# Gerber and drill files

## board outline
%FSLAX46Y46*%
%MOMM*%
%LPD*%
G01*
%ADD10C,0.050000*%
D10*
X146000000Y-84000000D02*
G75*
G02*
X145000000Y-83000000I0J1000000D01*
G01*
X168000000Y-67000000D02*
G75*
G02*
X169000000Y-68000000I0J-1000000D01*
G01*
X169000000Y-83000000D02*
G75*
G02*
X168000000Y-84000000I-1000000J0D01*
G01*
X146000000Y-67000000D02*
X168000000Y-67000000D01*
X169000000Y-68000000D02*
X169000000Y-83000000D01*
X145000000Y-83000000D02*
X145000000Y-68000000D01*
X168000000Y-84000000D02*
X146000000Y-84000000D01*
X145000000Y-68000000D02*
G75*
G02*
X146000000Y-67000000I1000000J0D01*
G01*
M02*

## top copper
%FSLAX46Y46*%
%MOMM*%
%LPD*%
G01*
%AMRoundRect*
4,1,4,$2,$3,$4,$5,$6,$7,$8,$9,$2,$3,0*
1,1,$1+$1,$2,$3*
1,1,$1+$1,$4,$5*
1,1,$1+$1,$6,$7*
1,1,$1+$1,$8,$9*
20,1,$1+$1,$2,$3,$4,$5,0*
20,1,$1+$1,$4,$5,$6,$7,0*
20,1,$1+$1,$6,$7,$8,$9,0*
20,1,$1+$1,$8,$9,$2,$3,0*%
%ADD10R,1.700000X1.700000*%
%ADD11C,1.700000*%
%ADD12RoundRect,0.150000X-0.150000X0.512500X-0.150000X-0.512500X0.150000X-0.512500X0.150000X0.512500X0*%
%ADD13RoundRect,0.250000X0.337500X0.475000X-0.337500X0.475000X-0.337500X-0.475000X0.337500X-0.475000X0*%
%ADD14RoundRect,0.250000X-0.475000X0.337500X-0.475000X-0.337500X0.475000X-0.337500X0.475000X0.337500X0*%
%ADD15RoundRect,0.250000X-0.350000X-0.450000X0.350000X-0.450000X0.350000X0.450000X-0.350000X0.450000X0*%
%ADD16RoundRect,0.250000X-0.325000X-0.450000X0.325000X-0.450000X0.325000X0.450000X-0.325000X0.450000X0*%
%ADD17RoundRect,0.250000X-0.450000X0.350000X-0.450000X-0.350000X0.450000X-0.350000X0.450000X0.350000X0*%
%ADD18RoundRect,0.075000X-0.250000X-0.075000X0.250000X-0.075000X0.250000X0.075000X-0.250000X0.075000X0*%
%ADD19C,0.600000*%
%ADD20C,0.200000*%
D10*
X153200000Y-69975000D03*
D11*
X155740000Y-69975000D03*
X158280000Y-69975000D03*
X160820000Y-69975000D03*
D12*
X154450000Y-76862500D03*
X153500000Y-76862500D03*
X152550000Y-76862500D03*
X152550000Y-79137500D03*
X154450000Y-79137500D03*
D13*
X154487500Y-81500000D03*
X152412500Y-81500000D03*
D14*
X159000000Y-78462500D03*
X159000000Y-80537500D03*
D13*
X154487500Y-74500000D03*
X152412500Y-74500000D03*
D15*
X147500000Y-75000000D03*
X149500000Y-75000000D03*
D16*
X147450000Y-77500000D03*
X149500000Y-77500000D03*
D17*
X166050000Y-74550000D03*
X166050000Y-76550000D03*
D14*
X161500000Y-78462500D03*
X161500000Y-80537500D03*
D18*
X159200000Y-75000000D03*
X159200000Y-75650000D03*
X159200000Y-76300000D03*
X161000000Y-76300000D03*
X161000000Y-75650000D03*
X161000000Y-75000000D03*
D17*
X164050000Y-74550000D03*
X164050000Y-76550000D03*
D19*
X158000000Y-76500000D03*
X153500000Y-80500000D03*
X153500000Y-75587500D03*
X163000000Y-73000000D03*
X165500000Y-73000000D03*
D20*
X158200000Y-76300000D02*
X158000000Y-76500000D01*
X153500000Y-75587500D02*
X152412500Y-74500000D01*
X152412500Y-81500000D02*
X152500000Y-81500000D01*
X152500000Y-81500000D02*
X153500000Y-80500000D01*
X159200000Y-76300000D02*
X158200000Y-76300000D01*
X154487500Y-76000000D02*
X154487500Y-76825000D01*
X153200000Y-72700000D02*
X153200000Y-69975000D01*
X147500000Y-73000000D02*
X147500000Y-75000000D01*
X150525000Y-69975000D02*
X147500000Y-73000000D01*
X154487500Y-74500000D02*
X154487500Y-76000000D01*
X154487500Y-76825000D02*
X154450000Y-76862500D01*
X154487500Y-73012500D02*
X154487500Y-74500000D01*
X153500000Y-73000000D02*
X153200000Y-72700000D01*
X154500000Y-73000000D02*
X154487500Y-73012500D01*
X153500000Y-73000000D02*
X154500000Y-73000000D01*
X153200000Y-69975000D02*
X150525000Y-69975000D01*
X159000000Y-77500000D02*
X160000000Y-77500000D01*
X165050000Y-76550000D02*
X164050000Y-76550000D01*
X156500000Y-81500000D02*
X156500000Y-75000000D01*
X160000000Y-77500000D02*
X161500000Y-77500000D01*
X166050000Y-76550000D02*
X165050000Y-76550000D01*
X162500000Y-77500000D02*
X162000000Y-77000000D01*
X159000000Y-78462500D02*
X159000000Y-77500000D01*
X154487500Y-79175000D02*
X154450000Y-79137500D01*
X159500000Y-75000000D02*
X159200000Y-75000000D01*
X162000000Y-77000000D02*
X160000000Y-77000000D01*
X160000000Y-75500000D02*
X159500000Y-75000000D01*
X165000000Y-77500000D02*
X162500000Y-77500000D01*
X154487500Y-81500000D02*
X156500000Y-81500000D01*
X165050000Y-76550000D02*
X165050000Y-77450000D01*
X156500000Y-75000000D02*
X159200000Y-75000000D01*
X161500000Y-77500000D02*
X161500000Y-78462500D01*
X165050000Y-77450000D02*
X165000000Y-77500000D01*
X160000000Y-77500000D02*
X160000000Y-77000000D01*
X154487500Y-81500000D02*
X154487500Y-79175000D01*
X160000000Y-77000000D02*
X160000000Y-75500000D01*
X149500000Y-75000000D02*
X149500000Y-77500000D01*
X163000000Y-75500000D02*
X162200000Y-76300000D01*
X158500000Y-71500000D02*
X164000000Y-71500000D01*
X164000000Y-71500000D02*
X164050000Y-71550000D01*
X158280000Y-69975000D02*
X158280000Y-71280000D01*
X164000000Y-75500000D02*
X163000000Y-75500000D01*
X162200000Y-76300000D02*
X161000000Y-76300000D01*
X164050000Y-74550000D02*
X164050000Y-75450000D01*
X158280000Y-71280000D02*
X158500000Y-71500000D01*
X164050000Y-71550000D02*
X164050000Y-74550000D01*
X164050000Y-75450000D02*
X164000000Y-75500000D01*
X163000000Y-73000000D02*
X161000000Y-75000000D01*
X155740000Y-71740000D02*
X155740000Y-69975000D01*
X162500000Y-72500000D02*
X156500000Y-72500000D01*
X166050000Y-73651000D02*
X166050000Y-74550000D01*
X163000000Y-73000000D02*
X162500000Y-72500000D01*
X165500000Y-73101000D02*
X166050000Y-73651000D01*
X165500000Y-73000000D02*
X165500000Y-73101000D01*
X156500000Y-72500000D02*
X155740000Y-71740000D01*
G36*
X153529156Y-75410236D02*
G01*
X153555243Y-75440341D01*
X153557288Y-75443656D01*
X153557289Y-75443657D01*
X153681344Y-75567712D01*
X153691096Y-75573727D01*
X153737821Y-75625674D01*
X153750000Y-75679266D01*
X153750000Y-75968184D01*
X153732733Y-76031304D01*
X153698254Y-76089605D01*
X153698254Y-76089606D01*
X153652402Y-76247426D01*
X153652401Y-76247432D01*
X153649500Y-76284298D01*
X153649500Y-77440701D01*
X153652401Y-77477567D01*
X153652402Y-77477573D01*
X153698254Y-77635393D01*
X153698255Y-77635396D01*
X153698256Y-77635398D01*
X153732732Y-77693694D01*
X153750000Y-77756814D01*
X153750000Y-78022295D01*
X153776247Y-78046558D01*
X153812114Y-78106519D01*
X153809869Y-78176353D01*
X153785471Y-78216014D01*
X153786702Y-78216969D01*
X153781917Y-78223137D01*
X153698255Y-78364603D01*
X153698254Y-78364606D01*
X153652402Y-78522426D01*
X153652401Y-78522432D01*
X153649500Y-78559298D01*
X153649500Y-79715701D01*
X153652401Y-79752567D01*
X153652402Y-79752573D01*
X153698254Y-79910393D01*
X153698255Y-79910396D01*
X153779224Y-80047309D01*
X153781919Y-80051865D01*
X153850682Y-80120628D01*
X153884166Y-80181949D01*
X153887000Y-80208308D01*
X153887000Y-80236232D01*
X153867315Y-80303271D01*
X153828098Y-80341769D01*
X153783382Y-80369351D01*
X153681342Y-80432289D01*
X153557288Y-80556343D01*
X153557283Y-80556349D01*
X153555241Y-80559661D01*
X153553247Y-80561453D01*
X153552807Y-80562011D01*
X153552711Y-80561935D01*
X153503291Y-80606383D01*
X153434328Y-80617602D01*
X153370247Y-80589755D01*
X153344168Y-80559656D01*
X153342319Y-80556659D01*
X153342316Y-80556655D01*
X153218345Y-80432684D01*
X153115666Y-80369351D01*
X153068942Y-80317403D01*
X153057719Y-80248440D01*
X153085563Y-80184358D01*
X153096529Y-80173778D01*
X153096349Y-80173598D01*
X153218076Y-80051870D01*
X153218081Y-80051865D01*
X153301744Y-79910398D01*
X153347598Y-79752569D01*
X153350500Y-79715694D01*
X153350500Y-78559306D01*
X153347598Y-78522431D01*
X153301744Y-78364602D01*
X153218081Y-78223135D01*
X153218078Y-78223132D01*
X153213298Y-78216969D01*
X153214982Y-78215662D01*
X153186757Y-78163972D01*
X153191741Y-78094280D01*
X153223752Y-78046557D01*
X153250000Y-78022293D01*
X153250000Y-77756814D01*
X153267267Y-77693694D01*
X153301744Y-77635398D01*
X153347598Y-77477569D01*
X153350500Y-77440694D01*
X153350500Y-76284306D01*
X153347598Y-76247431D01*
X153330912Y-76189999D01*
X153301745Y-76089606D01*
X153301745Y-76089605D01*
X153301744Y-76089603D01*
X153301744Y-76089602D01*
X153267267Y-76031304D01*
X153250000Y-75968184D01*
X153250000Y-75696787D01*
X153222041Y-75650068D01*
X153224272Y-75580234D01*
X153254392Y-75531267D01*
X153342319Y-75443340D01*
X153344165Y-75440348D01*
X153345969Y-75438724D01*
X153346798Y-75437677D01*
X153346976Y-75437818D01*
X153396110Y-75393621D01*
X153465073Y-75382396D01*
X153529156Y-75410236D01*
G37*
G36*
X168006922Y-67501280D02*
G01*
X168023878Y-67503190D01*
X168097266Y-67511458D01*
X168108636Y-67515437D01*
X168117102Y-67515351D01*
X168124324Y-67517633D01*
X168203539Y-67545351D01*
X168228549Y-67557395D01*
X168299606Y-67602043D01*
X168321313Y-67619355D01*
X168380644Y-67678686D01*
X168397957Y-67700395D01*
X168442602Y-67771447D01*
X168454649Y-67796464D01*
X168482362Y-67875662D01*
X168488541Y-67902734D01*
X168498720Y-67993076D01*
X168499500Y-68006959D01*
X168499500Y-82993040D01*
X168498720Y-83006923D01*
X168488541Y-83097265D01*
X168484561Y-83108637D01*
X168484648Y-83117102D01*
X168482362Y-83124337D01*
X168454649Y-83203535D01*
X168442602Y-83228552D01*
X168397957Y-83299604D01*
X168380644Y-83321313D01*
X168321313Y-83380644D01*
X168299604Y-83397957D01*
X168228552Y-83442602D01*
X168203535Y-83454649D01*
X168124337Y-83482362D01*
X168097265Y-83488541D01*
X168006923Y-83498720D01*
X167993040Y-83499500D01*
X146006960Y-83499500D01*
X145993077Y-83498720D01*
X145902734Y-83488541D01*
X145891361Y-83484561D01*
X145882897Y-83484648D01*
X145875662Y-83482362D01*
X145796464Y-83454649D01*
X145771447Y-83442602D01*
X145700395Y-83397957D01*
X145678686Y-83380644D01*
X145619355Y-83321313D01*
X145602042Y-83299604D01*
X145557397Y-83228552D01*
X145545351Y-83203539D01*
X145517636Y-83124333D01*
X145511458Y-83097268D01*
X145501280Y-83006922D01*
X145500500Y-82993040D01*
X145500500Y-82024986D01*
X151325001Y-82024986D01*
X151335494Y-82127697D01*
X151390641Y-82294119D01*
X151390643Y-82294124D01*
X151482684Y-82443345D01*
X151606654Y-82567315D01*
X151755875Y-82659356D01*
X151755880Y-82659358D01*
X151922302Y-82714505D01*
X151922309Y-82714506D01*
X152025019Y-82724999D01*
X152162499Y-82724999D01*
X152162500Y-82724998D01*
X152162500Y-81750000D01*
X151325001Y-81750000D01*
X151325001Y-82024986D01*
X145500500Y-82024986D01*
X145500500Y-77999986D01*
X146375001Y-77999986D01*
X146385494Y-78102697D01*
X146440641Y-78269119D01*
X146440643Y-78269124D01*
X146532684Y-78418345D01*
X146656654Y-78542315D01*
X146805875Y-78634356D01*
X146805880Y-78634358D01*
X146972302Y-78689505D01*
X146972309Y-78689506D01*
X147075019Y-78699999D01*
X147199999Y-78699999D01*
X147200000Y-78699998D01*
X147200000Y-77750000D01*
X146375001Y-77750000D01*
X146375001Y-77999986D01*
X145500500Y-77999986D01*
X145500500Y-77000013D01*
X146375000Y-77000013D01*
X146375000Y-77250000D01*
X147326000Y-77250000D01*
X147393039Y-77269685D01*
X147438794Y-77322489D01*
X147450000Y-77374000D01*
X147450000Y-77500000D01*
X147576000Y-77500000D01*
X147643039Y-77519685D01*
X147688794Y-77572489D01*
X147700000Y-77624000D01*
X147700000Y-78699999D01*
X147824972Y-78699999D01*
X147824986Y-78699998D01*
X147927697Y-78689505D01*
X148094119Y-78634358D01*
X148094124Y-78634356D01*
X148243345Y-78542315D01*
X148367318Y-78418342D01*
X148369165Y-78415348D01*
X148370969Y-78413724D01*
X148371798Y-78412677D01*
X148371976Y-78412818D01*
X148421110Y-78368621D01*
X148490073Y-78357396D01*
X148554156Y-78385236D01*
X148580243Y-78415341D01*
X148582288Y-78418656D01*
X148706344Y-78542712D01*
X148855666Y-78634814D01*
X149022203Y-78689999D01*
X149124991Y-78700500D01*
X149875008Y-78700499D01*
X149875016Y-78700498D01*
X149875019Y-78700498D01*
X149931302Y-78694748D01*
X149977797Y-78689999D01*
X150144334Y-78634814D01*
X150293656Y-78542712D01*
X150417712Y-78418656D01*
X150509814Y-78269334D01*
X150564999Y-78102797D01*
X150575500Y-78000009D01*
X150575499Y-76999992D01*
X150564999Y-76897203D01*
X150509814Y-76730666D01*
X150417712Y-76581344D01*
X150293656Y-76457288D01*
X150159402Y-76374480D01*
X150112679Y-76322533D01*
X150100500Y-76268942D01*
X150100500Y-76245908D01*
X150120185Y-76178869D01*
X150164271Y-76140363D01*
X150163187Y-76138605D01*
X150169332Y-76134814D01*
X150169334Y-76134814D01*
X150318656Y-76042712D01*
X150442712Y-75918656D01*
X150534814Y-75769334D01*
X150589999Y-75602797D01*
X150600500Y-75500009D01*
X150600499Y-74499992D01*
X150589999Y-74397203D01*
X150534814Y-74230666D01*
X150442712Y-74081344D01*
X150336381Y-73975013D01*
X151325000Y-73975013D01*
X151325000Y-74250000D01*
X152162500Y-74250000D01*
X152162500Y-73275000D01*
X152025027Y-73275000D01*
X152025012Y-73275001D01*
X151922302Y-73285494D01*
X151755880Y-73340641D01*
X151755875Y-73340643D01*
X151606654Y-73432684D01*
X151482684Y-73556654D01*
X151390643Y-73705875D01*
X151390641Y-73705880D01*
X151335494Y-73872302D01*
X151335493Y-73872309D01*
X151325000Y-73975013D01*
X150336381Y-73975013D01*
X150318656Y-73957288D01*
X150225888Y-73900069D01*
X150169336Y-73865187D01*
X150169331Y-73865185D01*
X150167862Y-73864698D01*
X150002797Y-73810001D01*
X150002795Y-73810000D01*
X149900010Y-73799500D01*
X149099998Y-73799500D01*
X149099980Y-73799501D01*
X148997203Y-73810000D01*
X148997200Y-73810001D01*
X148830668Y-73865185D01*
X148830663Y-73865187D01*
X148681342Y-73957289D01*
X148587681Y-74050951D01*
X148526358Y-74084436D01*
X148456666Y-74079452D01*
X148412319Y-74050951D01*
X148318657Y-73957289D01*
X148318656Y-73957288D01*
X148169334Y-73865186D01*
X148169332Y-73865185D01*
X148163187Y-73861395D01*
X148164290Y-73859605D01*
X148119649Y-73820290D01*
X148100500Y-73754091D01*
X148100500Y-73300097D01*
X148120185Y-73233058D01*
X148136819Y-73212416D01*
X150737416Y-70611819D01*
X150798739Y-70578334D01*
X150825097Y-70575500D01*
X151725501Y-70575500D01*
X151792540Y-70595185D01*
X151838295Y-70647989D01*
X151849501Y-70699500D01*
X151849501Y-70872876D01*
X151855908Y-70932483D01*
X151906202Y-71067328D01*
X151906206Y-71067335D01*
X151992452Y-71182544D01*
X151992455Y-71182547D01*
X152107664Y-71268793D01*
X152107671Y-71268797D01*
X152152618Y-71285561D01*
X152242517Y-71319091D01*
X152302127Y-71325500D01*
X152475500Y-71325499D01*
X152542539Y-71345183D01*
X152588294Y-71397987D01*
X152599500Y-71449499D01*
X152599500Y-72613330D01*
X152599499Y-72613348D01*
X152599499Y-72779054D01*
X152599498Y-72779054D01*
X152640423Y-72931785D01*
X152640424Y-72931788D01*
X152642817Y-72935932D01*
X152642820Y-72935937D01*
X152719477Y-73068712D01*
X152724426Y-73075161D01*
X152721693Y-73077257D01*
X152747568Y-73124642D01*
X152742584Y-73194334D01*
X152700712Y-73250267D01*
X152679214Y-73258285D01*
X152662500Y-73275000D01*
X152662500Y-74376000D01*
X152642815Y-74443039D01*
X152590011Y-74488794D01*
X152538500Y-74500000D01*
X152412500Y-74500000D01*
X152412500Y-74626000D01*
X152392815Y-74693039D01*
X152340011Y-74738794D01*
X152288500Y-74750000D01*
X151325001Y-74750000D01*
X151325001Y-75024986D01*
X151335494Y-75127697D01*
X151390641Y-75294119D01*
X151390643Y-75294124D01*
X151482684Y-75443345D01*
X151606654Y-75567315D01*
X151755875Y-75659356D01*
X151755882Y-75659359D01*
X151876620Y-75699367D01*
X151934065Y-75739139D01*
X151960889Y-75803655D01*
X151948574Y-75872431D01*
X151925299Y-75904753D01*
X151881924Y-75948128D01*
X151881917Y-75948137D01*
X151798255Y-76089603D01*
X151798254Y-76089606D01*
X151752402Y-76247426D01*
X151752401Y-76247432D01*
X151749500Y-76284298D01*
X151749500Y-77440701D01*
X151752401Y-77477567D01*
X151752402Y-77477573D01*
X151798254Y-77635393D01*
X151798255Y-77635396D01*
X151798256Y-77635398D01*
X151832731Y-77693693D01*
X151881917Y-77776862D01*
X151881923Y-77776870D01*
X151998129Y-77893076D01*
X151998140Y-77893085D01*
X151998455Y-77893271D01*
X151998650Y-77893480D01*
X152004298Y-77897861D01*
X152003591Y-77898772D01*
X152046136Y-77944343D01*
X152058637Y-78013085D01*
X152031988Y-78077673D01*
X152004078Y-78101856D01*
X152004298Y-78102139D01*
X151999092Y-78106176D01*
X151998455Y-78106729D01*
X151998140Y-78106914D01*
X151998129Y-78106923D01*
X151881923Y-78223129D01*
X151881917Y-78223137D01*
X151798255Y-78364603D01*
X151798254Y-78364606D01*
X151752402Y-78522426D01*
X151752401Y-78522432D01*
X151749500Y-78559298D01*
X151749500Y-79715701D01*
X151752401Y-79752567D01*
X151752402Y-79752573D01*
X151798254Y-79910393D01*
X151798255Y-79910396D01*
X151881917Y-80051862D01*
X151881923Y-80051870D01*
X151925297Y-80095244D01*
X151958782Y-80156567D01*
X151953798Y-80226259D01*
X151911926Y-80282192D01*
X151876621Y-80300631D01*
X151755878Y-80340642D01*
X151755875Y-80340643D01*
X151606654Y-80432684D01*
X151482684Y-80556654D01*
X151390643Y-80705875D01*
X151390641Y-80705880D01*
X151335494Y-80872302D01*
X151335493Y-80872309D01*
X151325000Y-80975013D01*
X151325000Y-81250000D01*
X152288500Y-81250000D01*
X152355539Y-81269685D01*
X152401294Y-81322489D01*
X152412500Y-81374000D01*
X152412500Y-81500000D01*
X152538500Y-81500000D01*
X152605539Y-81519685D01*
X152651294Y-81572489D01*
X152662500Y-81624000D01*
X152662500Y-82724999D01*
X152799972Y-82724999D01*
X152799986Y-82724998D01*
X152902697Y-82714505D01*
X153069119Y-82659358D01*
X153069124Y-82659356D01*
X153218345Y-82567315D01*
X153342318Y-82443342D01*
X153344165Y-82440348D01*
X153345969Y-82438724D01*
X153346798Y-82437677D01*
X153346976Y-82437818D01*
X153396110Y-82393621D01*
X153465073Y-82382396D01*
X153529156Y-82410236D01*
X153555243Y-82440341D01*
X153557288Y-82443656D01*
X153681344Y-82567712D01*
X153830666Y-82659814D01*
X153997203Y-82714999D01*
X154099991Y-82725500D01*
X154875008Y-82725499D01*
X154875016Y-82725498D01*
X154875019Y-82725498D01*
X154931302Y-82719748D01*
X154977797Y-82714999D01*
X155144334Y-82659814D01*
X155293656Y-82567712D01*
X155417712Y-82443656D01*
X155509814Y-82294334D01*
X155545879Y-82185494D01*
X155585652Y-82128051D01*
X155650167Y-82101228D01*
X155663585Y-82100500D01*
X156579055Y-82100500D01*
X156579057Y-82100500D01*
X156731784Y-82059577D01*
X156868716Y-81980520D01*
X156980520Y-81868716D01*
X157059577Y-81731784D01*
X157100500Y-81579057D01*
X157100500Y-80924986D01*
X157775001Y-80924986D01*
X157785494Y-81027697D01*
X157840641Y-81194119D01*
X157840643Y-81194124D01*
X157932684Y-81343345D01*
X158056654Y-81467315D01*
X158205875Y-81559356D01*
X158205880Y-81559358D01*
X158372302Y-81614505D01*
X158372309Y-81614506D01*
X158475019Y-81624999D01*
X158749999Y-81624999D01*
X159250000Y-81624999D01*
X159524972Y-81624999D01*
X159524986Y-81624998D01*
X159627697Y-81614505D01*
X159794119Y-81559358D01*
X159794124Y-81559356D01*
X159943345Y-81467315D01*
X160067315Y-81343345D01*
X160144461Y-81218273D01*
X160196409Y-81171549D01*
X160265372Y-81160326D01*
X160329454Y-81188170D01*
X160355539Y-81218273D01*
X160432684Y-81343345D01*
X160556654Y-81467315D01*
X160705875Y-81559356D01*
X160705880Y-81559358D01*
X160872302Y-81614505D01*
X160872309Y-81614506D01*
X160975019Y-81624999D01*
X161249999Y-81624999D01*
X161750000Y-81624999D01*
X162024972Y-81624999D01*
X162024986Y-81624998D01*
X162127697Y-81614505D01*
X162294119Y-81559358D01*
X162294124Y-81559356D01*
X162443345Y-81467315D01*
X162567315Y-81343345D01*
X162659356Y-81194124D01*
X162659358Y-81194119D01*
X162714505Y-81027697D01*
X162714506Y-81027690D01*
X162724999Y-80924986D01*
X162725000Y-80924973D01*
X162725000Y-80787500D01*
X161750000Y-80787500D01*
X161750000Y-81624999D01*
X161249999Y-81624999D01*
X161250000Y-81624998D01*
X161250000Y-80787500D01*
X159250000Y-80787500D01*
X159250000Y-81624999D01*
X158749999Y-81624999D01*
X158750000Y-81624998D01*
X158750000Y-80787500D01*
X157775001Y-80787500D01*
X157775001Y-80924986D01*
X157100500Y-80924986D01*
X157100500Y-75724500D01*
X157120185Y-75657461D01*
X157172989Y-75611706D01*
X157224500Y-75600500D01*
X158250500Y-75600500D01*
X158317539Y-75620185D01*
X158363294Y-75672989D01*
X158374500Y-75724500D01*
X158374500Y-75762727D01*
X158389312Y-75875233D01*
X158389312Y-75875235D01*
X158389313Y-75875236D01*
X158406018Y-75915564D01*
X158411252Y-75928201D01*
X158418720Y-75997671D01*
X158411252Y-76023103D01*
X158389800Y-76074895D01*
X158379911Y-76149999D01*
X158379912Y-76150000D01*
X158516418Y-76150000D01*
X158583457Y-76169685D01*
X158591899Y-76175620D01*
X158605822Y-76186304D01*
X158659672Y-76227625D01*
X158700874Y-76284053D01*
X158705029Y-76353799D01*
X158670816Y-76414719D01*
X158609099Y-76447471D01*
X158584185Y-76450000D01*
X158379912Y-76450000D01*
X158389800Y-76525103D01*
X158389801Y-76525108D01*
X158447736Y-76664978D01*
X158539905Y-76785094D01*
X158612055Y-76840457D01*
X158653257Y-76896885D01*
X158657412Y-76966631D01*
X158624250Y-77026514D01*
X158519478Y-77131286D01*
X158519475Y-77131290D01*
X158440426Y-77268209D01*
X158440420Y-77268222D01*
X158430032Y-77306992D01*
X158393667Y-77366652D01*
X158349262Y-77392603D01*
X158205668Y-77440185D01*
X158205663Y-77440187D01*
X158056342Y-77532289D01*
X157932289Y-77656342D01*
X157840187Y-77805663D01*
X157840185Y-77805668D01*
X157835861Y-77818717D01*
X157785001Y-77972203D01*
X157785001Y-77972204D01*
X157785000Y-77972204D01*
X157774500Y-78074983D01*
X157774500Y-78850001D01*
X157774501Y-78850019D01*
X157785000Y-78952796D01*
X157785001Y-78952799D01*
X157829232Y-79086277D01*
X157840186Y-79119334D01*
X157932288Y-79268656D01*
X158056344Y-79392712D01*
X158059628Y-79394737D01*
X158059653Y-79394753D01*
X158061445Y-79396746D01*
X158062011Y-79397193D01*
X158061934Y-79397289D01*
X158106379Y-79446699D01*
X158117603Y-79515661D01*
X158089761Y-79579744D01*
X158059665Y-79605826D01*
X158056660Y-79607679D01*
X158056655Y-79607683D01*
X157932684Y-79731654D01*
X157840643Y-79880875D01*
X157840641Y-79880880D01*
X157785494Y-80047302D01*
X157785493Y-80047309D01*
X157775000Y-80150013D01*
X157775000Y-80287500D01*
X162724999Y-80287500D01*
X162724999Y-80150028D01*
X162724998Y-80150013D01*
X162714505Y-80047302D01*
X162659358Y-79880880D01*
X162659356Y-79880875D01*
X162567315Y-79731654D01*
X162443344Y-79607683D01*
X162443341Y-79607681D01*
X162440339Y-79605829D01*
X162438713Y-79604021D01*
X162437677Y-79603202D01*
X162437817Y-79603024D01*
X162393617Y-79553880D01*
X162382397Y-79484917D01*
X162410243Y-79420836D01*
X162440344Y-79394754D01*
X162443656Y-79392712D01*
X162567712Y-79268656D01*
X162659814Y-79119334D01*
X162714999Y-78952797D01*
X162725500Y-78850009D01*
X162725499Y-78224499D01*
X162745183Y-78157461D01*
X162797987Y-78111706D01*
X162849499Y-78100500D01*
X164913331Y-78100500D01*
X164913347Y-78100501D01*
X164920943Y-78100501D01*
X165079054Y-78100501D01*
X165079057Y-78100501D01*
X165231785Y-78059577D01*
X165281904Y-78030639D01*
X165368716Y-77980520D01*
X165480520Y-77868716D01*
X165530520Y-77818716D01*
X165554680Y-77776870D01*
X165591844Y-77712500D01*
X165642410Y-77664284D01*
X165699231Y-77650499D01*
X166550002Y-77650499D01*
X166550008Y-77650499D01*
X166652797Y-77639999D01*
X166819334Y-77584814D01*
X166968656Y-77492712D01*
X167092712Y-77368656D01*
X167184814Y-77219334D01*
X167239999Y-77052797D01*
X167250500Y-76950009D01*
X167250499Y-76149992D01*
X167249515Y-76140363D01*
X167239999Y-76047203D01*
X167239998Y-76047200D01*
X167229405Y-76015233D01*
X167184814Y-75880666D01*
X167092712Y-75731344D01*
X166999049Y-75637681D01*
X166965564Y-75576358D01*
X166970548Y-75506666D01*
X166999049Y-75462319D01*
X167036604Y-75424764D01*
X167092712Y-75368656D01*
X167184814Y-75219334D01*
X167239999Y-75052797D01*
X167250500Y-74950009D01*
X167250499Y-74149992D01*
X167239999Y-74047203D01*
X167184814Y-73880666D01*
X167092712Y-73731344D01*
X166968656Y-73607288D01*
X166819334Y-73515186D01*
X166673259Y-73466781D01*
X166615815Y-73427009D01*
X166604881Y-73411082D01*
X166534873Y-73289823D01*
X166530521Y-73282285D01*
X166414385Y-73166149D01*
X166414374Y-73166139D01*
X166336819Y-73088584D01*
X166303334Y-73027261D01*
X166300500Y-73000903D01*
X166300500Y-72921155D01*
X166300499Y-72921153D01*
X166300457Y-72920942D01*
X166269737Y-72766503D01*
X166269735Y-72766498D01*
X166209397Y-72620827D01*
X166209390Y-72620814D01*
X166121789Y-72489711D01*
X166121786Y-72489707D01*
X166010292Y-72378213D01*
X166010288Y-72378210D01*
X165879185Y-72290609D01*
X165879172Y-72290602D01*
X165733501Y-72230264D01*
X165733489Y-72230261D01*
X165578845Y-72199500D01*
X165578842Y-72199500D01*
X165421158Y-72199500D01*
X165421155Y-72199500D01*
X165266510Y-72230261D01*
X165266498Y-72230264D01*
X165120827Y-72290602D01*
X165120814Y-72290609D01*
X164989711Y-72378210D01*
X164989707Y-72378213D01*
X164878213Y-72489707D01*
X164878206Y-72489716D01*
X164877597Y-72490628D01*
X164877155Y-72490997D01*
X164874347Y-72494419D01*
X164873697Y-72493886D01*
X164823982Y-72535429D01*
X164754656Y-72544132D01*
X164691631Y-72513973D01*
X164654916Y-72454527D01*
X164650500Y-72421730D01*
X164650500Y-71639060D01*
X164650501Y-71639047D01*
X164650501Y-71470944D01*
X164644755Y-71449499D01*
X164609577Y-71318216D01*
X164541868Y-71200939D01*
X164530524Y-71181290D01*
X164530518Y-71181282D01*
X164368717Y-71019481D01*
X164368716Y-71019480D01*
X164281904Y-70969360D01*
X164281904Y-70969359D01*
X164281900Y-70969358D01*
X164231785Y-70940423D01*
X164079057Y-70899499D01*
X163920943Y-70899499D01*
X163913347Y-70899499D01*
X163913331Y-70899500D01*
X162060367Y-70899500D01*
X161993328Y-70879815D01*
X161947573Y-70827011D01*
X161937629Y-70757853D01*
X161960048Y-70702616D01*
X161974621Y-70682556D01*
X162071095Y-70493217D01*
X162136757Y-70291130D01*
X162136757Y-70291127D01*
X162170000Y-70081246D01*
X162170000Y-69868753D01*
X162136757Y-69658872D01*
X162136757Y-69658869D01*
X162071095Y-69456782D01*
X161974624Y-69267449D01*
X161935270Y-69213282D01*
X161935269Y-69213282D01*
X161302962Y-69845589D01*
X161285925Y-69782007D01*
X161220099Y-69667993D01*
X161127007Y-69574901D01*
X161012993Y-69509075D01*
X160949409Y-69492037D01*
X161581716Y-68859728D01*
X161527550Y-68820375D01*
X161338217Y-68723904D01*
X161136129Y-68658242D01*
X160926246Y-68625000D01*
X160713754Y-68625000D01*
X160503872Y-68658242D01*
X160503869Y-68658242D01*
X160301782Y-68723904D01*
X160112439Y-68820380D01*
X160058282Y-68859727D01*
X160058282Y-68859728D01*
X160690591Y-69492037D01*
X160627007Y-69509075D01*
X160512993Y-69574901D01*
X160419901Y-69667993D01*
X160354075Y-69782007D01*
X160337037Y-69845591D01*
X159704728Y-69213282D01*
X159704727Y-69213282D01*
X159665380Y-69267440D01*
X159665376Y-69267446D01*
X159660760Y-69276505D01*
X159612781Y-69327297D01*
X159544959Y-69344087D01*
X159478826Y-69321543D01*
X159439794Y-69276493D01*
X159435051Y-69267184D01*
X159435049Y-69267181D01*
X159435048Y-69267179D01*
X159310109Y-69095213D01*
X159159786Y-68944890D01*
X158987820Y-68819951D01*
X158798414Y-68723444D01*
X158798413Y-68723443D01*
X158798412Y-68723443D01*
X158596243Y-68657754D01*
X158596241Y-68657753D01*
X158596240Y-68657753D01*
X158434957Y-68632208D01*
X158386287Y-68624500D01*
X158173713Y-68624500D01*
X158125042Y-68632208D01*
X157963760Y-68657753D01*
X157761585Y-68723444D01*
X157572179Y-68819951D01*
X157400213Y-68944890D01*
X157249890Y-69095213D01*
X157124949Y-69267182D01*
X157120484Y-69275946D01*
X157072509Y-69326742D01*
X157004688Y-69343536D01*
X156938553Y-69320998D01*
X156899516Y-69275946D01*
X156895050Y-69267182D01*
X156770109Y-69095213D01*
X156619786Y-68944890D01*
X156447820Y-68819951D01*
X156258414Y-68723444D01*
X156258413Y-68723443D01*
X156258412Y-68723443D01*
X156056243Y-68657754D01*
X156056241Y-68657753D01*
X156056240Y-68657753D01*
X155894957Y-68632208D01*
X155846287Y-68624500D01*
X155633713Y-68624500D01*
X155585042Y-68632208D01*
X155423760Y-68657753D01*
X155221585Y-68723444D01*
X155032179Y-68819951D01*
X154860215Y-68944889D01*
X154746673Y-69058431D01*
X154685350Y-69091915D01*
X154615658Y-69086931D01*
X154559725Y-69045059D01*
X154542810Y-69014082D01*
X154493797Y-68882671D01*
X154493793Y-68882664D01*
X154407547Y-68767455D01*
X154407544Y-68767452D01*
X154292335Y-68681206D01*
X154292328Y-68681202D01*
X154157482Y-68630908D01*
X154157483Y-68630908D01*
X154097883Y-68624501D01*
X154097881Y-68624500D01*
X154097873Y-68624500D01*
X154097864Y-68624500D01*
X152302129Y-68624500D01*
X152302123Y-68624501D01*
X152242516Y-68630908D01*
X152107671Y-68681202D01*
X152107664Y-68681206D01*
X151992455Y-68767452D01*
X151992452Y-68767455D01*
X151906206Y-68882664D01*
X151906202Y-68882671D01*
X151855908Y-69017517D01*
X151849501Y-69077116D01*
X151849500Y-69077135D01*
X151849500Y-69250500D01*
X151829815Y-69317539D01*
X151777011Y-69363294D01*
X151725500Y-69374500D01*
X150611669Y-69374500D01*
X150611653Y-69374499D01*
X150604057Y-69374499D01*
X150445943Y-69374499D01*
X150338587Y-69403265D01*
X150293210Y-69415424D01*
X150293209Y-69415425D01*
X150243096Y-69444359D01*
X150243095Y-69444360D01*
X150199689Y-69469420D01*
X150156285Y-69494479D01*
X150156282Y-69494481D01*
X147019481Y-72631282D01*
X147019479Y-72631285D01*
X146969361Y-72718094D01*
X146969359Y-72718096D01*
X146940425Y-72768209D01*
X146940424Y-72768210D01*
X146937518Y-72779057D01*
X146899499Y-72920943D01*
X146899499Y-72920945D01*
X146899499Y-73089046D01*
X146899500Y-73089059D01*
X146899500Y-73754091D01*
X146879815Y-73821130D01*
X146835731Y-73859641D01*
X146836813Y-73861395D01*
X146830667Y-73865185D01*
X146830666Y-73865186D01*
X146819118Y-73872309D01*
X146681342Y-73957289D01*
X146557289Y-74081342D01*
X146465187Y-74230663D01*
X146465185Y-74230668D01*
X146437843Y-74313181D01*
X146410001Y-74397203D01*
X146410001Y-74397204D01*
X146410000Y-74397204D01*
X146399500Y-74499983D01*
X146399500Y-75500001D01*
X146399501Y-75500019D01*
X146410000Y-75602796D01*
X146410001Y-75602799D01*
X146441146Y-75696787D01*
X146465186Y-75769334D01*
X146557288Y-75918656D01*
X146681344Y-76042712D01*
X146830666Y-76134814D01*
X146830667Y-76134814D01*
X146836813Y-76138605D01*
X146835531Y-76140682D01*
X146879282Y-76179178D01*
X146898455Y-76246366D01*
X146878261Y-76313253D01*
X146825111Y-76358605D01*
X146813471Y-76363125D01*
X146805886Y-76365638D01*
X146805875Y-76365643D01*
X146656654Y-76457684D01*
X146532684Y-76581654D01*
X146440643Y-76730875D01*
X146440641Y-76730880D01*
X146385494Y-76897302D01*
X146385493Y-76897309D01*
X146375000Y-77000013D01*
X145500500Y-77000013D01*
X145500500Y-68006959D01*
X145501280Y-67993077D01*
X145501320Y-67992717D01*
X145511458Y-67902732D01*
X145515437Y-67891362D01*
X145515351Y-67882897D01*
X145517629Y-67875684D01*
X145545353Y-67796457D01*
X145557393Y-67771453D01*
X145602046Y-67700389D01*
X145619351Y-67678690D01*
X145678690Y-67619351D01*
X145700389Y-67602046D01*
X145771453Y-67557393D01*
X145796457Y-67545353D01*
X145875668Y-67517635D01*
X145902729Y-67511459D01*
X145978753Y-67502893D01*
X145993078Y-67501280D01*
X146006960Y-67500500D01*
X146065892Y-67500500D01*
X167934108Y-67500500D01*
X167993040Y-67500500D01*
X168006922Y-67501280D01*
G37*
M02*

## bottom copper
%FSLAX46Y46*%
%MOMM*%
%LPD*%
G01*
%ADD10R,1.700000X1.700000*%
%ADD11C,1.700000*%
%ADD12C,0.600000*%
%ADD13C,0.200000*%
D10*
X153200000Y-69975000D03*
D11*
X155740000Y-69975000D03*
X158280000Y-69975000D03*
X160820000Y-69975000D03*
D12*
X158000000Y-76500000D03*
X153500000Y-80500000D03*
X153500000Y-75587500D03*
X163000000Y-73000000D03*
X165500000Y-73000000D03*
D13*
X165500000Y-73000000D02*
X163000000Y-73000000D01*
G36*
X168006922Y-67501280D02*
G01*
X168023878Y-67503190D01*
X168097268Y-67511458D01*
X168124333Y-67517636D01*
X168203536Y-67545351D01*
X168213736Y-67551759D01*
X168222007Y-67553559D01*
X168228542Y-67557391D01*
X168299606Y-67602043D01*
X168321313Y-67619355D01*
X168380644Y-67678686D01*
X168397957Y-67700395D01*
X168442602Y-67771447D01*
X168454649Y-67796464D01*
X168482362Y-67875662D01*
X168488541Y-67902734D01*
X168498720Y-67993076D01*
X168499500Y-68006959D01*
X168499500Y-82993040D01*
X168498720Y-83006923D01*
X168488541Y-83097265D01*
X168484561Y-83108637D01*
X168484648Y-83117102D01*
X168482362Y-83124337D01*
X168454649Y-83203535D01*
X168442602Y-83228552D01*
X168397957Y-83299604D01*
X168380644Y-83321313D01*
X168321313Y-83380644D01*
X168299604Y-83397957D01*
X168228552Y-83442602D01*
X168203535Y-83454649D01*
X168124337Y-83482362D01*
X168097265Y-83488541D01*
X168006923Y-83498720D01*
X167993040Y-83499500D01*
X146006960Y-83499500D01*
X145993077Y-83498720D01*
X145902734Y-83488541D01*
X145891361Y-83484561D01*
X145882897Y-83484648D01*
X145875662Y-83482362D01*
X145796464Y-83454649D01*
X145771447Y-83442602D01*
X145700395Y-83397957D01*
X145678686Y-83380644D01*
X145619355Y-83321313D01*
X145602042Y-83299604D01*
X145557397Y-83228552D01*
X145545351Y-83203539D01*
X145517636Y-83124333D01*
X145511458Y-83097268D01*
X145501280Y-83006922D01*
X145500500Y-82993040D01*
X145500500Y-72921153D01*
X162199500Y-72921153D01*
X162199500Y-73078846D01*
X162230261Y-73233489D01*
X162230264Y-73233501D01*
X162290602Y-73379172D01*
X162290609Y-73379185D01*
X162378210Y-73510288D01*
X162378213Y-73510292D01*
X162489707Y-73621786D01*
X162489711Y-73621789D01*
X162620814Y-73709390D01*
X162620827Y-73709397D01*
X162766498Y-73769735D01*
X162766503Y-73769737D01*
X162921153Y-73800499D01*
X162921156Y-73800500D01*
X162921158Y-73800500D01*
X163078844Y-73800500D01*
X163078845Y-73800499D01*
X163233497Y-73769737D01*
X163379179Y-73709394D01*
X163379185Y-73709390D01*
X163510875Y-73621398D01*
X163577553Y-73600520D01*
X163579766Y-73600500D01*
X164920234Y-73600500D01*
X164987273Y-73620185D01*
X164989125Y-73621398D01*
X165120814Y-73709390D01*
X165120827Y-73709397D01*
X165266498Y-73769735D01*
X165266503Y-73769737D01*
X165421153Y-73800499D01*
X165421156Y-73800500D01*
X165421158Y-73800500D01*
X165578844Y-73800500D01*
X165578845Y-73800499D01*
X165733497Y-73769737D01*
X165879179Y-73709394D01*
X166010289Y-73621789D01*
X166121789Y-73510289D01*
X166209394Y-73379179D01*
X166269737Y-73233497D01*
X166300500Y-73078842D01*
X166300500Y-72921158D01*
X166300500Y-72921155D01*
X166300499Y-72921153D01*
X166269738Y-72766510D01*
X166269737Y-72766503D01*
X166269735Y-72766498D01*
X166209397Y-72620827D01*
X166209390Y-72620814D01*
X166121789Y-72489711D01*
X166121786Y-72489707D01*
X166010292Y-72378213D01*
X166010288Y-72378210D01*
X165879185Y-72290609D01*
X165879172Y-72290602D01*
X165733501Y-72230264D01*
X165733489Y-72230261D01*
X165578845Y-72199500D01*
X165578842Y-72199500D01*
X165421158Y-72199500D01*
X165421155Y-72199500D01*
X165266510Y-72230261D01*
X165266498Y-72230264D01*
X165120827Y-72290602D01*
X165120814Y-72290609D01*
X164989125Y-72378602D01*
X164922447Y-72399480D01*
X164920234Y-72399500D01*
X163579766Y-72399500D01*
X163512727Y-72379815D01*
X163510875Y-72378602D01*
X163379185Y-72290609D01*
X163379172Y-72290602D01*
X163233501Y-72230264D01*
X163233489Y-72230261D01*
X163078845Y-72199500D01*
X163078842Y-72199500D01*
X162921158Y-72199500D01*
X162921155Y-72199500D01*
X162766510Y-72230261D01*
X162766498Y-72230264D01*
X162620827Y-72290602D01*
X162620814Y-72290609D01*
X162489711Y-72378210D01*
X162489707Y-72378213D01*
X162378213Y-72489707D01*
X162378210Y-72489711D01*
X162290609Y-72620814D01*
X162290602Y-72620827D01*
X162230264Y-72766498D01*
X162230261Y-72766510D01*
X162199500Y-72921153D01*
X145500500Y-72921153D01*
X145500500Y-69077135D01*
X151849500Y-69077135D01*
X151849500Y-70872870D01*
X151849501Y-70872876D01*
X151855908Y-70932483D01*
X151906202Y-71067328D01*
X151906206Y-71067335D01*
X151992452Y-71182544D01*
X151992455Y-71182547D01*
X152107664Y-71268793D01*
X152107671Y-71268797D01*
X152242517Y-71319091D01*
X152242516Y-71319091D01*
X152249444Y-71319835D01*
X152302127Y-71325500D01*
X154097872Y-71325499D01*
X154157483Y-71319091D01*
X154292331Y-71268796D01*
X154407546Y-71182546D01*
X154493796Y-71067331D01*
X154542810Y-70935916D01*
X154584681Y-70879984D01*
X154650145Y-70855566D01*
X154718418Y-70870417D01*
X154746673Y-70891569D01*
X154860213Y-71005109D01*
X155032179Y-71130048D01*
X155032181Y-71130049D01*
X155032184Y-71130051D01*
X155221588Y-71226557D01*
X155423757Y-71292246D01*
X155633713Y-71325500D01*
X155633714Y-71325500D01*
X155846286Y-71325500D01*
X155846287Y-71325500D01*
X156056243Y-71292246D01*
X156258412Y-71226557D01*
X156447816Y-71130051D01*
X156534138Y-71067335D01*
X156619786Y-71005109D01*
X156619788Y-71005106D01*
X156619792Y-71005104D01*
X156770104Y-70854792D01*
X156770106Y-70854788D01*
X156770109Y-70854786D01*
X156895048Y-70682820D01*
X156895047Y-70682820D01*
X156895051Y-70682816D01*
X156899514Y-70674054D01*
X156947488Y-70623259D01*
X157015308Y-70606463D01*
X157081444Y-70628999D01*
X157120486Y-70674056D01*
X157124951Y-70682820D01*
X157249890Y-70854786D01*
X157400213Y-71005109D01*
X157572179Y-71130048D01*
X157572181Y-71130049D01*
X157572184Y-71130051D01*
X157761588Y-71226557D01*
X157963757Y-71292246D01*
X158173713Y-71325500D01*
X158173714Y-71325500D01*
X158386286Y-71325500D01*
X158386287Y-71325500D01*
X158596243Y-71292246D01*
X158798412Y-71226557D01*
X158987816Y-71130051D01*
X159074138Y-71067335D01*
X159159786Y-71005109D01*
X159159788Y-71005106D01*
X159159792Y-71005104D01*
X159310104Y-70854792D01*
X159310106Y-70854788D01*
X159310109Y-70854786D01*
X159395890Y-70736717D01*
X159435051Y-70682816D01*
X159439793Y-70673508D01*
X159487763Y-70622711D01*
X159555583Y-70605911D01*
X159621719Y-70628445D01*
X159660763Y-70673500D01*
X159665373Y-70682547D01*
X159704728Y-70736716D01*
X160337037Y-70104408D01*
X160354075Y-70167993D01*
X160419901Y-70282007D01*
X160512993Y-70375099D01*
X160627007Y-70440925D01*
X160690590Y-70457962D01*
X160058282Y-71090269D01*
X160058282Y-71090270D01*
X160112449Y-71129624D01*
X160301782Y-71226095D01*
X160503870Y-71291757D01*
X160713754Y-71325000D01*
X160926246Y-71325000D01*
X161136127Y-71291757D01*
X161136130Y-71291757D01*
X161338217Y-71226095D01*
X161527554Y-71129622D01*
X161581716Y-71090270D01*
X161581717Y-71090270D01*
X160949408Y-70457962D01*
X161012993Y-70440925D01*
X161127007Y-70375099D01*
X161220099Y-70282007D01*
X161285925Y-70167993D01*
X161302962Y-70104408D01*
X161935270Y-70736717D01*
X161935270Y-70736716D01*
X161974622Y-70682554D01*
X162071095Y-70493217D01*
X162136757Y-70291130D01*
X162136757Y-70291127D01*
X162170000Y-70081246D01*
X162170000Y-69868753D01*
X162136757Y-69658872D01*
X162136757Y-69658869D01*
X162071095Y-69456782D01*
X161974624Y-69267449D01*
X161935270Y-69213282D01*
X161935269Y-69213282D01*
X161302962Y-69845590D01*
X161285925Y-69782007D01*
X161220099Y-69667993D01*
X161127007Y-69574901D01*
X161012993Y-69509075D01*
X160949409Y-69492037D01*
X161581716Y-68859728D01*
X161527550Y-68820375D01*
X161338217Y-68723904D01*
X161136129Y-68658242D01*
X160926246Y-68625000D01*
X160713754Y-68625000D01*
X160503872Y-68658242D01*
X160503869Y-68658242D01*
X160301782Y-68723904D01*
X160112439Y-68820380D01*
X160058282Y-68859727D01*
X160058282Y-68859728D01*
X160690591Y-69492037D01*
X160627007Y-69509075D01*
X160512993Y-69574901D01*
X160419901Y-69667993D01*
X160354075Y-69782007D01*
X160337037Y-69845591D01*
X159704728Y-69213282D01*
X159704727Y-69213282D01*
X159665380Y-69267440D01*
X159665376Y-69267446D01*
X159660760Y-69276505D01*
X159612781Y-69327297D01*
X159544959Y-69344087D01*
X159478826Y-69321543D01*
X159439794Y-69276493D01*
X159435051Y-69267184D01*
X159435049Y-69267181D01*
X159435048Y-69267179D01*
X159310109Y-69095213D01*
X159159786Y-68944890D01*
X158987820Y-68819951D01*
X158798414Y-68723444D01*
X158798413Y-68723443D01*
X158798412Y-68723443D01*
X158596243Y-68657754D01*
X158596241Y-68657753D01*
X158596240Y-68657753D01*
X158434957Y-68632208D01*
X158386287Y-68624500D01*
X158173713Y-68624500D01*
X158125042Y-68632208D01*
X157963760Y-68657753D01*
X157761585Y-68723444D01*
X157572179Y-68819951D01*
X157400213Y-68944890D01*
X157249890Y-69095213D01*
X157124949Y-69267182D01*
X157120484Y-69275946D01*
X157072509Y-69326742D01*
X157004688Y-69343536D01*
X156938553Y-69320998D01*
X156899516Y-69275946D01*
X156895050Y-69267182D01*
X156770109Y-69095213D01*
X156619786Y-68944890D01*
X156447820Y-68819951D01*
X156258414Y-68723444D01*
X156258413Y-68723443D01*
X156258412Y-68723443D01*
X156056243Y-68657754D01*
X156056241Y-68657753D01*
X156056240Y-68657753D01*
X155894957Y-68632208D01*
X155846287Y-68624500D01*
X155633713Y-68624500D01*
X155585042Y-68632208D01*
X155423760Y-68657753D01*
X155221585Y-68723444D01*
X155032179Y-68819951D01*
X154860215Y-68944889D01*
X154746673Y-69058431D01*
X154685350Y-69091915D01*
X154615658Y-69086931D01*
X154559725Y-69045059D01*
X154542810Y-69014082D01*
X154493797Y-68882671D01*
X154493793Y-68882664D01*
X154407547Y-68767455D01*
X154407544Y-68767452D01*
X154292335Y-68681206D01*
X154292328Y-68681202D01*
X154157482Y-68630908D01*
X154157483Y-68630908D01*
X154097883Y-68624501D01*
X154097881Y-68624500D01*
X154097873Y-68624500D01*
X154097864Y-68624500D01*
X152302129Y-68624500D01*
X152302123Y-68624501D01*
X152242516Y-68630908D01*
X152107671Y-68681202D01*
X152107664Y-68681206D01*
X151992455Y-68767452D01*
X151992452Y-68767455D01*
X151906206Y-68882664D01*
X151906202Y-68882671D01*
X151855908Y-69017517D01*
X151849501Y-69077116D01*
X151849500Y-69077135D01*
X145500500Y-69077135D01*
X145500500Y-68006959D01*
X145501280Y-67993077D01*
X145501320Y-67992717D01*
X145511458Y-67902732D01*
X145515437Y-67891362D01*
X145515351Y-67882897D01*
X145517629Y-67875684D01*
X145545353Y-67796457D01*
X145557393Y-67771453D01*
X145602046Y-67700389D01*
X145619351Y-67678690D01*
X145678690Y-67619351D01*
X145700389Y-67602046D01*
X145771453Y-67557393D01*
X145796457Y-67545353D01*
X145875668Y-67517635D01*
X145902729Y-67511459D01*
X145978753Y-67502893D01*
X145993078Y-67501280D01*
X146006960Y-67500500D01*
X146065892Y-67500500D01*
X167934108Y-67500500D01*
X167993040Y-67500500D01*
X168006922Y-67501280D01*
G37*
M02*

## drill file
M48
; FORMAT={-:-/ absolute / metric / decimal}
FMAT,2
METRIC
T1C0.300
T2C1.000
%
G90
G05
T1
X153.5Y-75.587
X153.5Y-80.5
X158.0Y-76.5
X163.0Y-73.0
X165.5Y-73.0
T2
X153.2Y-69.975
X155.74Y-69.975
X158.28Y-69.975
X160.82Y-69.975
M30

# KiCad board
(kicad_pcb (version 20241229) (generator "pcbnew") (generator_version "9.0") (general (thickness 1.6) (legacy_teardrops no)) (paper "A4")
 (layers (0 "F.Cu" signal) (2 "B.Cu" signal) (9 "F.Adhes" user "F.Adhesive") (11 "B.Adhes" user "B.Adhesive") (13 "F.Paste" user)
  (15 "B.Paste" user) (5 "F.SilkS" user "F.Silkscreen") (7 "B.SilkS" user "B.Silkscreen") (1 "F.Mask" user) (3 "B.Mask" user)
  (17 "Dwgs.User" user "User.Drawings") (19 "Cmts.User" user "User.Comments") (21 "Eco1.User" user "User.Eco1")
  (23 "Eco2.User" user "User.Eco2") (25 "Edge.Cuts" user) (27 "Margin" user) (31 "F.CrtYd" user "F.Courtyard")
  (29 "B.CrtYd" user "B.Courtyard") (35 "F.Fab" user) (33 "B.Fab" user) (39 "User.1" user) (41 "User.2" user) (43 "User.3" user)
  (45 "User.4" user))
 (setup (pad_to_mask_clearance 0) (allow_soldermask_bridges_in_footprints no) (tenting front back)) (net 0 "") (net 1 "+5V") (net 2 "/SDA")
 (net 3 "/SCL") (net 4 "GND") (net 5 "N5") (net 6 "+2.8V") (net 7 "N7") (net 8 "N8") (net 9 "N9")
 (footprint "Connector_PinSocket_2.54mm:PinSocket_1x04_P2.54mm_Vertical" (layer "F.Cu") (at 153.2 69.975 90)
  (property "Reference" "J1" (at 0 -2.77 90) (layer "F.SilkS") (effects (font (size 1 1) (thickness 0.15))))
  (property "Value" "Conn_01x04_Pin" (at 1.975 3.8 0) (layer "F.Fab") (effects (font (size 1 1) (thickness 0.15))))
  (pad "1" thru_hole rect (at 0 0 90) (size 1.7 1.7) (drill 1) (layers "*.Cu" "*.Mask") (remove_unused_layers no) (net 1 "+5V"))
  (pad "2" thru_hole circle (at 0 2.54 90) (size 1.7 1.7) (drill 1) (layers "*.Cu" "*.Mask") (remove_unused_layers no) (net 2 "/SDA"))
  (pad "3" thru_hole circle (at 0 5.08 90) (size 1.7 1.7) (drill 1) (layers "*.Cu" "*.Mask") (remove_unused_layers no) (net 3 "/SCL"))
  (pad "4" thru_hole circle (at 0 7.62 90) (size 1.7 1.7) (drill 1) (layers "*.Cu" "*.Mask") (remove_unused_layers no) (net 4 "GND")))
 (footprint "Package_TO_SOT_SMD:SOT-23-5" (layer "F.Cu") (at 153.5 78 -90)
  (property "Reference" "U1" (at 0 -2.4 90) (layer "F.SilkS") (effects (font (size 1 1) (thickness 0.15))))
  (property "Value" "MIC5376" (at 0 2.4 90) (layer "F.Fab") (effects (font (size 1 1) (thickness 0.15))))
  (pad "1" smd roundrect (at -1.1375 -0.95 270) (size 1.325 0.6) (layers "F.Cu" "F.Mask" "F.Paste") (roundrect_rratio 0.25) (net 1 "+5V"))
  (pad "2" smd roundrect (at -1.1375 0 270) (size 1.325 0.6) (layers "F.Cu" "F.Mask" "F.Paste") (roundrect_rratio 0.25) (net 4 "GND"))
  (pad "3" smd roundrect (at -1.1375 0.95 270) (size 1.325 0.6) (layers "F.Cu" "F.Mask" "F.Paste") (roundrect_rratio 0.25) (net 1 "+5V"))
  (pad "4" smd roundrect (at 1.1375 0.95 270) (size 1.325 0.6) (layers "F.Cu" "F.Mask" "F.Paste") (roundrect_rratio 0.25) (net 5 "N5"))
  (pad "5" smd roundrect (at 1.1375 -0.95 270) (size 1.325 0.6) (layers "F.Cu" "F.Mask" "F.Paste") (roundrect_rratio 0.25) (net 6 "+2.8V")))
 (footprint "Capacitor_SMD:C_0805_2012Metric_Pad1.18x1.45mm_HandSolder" (layer "F.Cu") (at 153.45 81.5 180)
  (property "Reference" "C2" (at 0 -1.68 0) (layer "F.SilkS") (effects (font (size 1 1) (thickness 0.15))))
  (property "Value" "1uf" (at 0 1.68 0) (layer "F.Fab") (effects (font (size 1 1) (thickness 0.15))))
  (pad "1" smd roundrect (at -1.0375 0 180) (size 1.175 1.45) (layers "F.Cu" "F.Mask" "F.Paste") (roundrect_rratio 0.212766) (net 6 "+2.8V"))
  (pad "2" smd roundrect (at 1.0375 0 180) (size 1.175 1.45) (layers "F.Cu" "F.Mask" "F.Paste") (roundrect_rratio 0.212766) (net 4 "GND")))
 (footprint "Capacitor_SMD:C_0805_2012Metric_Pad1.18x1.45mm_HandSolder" (layer "F.Cu") (at 159 79.5 -90)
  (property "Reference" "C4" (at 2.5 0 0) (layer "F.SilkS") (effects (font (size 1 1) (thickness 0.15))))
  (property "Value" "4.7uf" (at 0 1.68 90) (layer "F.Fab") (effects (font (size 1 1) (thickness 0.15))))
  (pad "1" smd roundrect (at -1.0375 0 270) (size 1.175 1.45) (layers "F.Cu" "F.Mask" "F.Paste") (roundrect_rratio 0.212766) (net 6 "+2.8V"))
  (pad "2" smd roundrect (at 1.0375 0 270) (size 1.175 1.45) (layers "F.Cu" "F.Mask" "F.Paste") (roundrect_rratio 0.212766) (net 4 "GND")))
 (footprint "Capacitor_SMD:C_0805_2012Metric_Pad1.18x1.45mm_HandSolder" (layer "F.Cu") (at 153.45 74.5 180)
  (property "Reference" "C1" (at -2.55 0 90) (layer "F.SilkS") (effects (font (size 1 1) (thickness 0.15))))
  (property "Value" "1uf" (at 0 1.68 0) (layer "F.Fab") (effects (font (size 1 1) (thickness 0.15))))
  (pad "1" smd roundrect (at -1.0375 0 180) (size 1.175 1.45) (layers "F.Cu" "F.Mask" "F.Paste") (roundrect_rratio 0.212766) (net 1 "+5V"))
  (pad "2" smd roundrect (at 1.0375 0 180) (size 1.175 1.45) (layers "F.Cu" "F.Mask" "F.Paste") (roundrect_rratio 0.212766) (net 4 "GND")))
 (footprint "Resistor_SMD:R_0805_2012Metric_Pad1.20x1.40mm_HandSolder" (layer "F.Cu") (at 148.5 75)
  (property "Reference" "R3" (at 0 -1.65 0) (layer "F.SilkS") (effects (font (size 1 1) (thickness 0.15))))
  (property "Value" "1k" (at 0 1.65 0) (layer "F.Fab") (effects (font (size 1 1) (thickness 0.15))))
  (pad "1" smd roundrect (at -1 0) (size 1.2 1.4) (layers "F.Cu" "F.Mask" "F.Paste") (roundrect_rratio 0.208333) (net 1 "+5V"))
  (pad "2" smd roundrect (at 1 0) (size 1.2 1.4) (layers "F.Cu" "F.Mask" "F.Paste") (roundrect_rratio 0.208333) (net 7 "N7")))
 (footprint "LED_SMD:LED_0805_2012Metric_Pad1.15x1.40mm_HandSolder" (layer "F.Cu") (at 148.475 77.5)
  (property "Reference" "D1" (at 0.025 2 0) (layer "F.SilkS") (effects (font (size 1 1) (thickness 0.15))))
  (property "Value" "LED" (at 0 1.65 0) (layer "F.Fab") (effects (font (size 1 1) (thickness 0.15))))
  (pad "1" smd roundrect (at -1.025 0) (size 1.15 1.4) (layers "F.Cu" "F.Mask" "F.Paste") (roundrect_rratio 0.217391) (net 4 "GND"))
  (pad "2" smd roundrect (at 1.025 0) (size 1.15 1.4) (layers "F.Cu" "F.Mask" "F.Paste") (roundrect_rratio 0.217391) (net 7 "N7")))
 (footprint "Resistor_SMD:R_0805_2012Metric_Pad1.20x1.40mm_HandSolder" (layer "F.Cu") (at 166.05 75.55 -90)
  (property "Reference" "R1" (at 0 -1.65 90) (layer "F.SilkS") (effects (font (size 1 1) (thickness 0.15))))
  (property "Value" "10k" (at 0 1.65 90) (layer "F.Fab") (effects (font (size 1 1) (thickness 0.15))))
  (pad "1" smd roundrect (at -1 0 270) (size 1.2 1.4) (layers "F.Cu" "F.Mask" "F.Paste") (roundrect_rratio 0.208333) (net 2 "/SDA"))
  (pad "2" smd roundrect (at 1 0 270) (size 1.2 1.4) (layers "F.Cu" "F.Mask" "F.Paste") (roundrect_rratio 0.208333) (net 6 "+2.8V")))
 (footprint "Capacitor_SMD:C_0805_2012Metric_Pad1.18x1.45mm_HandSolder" (layer "F.Cu") (at 161.5 79.5 -90)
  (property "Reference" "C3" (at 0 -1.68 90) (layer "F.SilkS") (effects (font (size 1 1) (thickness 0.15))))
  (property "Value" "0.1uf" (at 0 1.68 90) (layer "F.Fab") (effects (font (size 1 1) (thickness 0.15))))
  (pad "1" smd roundrect (at -1.0375 0 270) (size 1.175 1.45) (layers "F.Cu" "F.Mask" "F.Paste") (roundrect_rratio 0.212766) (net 6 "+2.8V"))
  (pad "2" smd roundrect (at 1.0375 0 270) (size 1.175 1.45) (layers "F.Cu" "F.Mask" "F.Paste") (roundrect_rratio 0.212766) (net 4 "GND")))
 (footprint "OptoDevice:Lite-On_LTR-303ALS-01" (layer "F.Cu") (at 160.1 75.65)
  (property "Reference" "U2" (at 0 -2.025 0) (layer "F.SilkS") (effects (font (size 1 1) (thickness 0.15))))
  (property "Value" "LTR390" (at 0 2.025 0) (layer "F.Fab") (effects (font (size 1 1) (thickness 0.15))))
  (pad "1" smd roundrect (at -0.9 -0.65) (size 0.65 0.3) (layers "F.Cu" "F.Mask" "F.Paste") (roundrect_rratio 0.25) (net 6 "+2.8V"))
  (pad "2" smd roundrect (at -0.9 0) (size 0.65 0.3) (layers "F.Cu" "F.Mask" "F.Paste") (roundrect_rratio 0.25) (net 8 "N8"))
  (pad "3" smd roundrect (at -0.9 0.65) (size 0.65 0.3) (layers "F.Cu" "F.Mask" "F.Paste") (roundrect_rratio 0.25) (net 4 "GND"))
  (pad "4" smd roundrect (at 0.9 0.65) (size 0.65 0.3) (layers "F.Cu" "F.Mask" "F.Paste") (roundrect_rratio 0.25) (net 3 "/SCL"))
  (pad "5" smd roundrect (at 0.9 0) (size 0.65 0.3) (layers "F.Cu" "F.Mask" "F.Paste") (roundrect_rratio 0.25) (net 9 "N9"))
  (pad "6" smd roundrect (at 0.9 -0.65) (size 0.65 0.3) (layers "F.Cu" "F.Mask" "F.Paste") (roundrect_rratio 0.25) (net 2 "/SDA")))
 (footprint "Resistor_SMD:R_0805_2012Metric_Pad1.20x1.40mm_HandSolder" (layer "F.Cu") (at 164.05 75.55 -90)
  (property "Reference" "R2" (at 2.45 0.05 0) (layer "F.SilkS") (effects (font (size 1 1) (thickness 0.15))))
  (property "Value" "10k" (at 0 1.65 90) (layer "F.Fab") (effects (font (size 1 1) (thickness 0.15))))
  (pad "1" smd roundrect (at -1 0 270) (size 1.2 1.4) (layers "F.Cu" "F.Mask" "F.Paste") (roundrect_rratio 0.208333) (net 3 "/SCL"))
  (pad "2" smd roundrect (at 1 0 270) (size 1.2 1.4) (layers "F.Cu" "F.Mask" "F.Paste") (roundrect_rratio 0.208333) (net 6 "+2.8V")))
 (gr_arc (start 146 84) (mid 145.292893 83.707107) (end 145 83) (stroke (width 0.05) (type default)) (layer "Edge.Cuts"))
 (gr_arc (start 168 67) (mid 168.707107 67.292893) (end 169 68) (stroke (width 0.05) (type default)) (layer "Edge.Cuts"))
 (gr_arc (start 169 83) (mid 168.707107 83.707107) (end 168 84) (stroke (width 0.05) (type default)) (layer "Edge.Cuts"))
 (gr_line (start 146 67) (end 168 67) (stroke (width 0.05) (type default)) (layer "Edge.Cuts"))
 (gr_line (start 169 68) (end 169 83) (stroke (width 0.05) (type default)) (layer "Edge.Cuts"))
 (gr_line (start 145 83) (end 145 68) (stroke (width 0.05) (type default)) (layer "Edge.Cuts"))
 (gr_line (start 168 84) (end 146 84) (stroke (width 0.05) (type default)) (layer "Edge.Cuts"))
 (gr_arc (start 145 68) (mid 145.292893 67.292893) (end 146 67) (stroke (width 0.05) (type default)) (layer "Edge.Cuts"))
 (segment (start 158.2 76.3) (end 158 76.5) (width 0.2) (layer "F.Cu") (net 4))
 (segment (start 153.5 75.5875) (end 152.4125 74.5) (width 0.2) (layer "F.Cu") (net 4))
 (segment (start 152.4125 81.5) (end 152.5 81.5) (width 0.2) (layer "F.Cu") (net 4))
 (segment (start 152.5 81.5) (end 153.5 80.5) (width 0.2) (layer "F.Cu") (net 4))
 (segment (start 159.2 76.3) (end 158.2 76.3) (width 0.2) (layer "F.Cu") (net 4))
 (via (at 158 76.5) (size 0.6) (drill 0.3) (layers "F.Cu" "B.Cu") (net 4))
 (via (at 153.5 80.5) (size 0.6) (drill 0.3) (layers "F.Cu" "B.Cu") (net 4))
 (via (at 153.5 75.5875) (size 0.6) (drill 0.3) (layers "F.Cu" "B.Cu") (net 4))
 (segment (start 154.4875 76) (end 154.4875 76.825) (width 0.2) (layer "F.Cu") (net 1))
 (segment (start 153.2 72.7) (end 153.2 69.975) (width 0.2) (layer "F.Cu") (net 1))
 (segment (start 147.5 73) (end 147.5 75) (width 0.2) (layer "F.Cu") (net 1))
 (segment (start 150.525 69.975) (end 147.5 73) (width 0.2) (layer "F.Cu") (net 1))
 (segment (start 154.4875 74.5) (end 154.4875 76) (width 0.2) (layer "F.Cu") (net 1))
 (segment (start 154.4875 76.825) (end 154.45 76.8625) (width 0.2) (layer "F.Cu") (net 1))
 (segment (start 154.4875 73.0125) (end 154.4875 74.5) (width 0.2) (layer "F.Cu") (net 1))
 (segment (start 153.5 73) (end 153.2 72.7) (width 0.2) (layer "F.Cu") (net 1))
 (segment (start 154.5 73) (end 154.4875 73.0125) (width 0.2) (layer "F.Cu") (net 1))
 (segment (start 153.5 73) (end 154.5 73) (width 0.2) (layer "F.Cu") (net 1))
 (segment (start 153.2 69.975) (end 150.525 69.975) (width 0.2) (layer "F.Cu") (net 1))
 (segment (start 159 77.5) (end 160 77.5) (width 0.2) (layer "F.Cu") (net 6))
 (segment (start 165.05 76.55) (end 164.05 76.55) (width 0.2) (layer "F.Cu") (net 6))
 (segment (start 156.5 81.5) (end 156.5 75) (width 0.2) (layer "F.Cu") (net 6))
 (segment (start 160 77.5) (end 161.5 77.5) (width 0.2) (layer "F.Cu") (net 6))
 (segment (start 166.05 76.55) (end 165.05 76.55) (width 0.2) (layer "F.Cu") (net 6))
 (segment (start 162.5 77.5) (end 162 77) (width 0.2) (layer "F.Cu") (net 6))
 (segment (start 159 78.4625) (end 159 77.5) (width 0.2) (layer "F.Cu") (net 6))
 (segment (start 154.4875 79.175) (end 154.45 79.1375) (width 0.2) (layer "F.Cu") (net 6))
 (segment (start 159.5 75) (end 159.2 75) (width 0.2) (layer "F.Cu") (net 6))
 (segment (start 162 77) (end 160 77) (width 0.2) (layer "F.Cu") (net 6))
 (segment (start 160 75.5) (end 159.5 75) (width 0.2) (layer "F.Cu") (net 6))
 (segment (start 165 77.5) (end 162.5 77.5) (width 0.2) (layer "F.Cu") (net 6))
 (segment (start 154.4875 81.5) (end 156.5 81.5) (width 0.2) (layer "F.Cu") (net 6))
 (segment (start 165.05 76.55) (end 165.05 77.45) (width 0.2) (layer "F.Cu") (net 6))
 (segment (start 156.5 75) (end 159.2 75) (width 0.2) (layer "F.Cu") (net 6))
 (segment (start 161.5 77.5) (end 161.5 78.4625) (width 0.2) (layer "F.Cu") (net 6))
 (segment (start 165.05 77.45) (end 165 77.5) (width 0.2) (layer "F.Cu") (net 6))
 (segment (start 160 77.5) (end 160 77) (width 0.2) (layer "F.Cu") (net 6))
 (segment (start 154.4875 81.5) (end 154.4875 79.175) (width 0.2) (layer "F.Cu") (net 6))
 (segment (start 160 77) (end 160 75.5) (width 0.2) (layer "F.Cu") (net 6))
 (segment (start 149.5 75) (end 149.5 77.5) (width 0.2) (layer "F.Cu") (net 7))
 (segment (start 163 75.5) (end 162.2 76.3) (width 0.2) (layer "F.Cu") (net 3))
 (segment (start 158.5 71.5) (end 164 71.5) (width 0.2) (layer "F.Cu") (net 3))
 (segment (start 164 71.5) (end 164.05 71.55) (width 0.2) (layer "F.Cu") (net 3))
 (segment (start 158.28 69.975) (end 158.28 71.28) (width 0.2) (layer "F.Cu") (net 3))
 (segment (start 164 75.5) (end 163 75.5) (width 0.2) (layer "F.Cu") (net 3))
 (segment (start 162.2 76.3) (end 161 76.3) (width 0.2) (layer "F.Cu") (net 3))
 (segment (start 164.05 74.55) (end 164.05 75.45) (width 0.2) (layer "F.Cu") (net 3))
 (segment (start 158.28 71.28) (end 158.5 71.5) (width 0.2) (layer "F.Cu") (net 3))
 (segment (start 164.05 71.55) (end 164.05 74.55) (width 0.2) (layer "F.Cu") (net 3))
 (segment (start 164.05 75.45) (end 164 75.5) (width 0.2) (layer "F.Cu") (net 3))
 (segment (start 163 73) (end 161 75) (width 0.2) (layer "F.Cu") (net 2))
 (segment (start 155.74 71.74) (end 155.74 69.975) (width 0.2) (layer "F.Cu") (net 2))
 (segment (start 162.5 72.5) (end 156.5 72.5) (width 0.2) (layer "F.Cu") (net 2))
 (segment (start 166.05 73.651) (end 166.05 74.55) (width 0.2) (layer "F.Cu") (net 2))
 (segment (start 163 73) (end 162.5 72.5) (width 0.2) (layer "F.Cu") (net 2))
 (segment (start 165.5 73.101) (end 166.05 73.651) (width 0.2) (layer "F.Cu") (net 2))
 (segment (start 165.5 73) (end 165.5 73.101) (width 0.2) (layer "F.Cu") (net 2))
 (segment (start 156.5 72.5) (end 155.74 71.74) (width 0.2) (layer "F.Cu") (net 2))
 (via (at 163 73) (size 0.6) (drill 0.3) (layers "F.Cu" "B.Cu") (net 2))
 (via (at 165.5 73) (size 0.6) (drill 0.3) (layers "F.Cu" "B.Cu") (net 2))
 (segment (start 165.5 73) (end 163 73) (width 0.2) (layer "B.Cu") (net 2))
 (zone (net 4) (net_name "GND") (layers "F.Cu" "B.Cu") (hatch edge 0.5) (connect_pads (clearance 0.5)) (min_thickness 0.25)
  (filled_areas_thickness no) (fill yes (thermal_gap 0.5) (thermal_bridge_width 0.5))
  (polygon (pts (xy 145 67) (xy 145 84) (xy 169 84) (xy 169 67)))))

